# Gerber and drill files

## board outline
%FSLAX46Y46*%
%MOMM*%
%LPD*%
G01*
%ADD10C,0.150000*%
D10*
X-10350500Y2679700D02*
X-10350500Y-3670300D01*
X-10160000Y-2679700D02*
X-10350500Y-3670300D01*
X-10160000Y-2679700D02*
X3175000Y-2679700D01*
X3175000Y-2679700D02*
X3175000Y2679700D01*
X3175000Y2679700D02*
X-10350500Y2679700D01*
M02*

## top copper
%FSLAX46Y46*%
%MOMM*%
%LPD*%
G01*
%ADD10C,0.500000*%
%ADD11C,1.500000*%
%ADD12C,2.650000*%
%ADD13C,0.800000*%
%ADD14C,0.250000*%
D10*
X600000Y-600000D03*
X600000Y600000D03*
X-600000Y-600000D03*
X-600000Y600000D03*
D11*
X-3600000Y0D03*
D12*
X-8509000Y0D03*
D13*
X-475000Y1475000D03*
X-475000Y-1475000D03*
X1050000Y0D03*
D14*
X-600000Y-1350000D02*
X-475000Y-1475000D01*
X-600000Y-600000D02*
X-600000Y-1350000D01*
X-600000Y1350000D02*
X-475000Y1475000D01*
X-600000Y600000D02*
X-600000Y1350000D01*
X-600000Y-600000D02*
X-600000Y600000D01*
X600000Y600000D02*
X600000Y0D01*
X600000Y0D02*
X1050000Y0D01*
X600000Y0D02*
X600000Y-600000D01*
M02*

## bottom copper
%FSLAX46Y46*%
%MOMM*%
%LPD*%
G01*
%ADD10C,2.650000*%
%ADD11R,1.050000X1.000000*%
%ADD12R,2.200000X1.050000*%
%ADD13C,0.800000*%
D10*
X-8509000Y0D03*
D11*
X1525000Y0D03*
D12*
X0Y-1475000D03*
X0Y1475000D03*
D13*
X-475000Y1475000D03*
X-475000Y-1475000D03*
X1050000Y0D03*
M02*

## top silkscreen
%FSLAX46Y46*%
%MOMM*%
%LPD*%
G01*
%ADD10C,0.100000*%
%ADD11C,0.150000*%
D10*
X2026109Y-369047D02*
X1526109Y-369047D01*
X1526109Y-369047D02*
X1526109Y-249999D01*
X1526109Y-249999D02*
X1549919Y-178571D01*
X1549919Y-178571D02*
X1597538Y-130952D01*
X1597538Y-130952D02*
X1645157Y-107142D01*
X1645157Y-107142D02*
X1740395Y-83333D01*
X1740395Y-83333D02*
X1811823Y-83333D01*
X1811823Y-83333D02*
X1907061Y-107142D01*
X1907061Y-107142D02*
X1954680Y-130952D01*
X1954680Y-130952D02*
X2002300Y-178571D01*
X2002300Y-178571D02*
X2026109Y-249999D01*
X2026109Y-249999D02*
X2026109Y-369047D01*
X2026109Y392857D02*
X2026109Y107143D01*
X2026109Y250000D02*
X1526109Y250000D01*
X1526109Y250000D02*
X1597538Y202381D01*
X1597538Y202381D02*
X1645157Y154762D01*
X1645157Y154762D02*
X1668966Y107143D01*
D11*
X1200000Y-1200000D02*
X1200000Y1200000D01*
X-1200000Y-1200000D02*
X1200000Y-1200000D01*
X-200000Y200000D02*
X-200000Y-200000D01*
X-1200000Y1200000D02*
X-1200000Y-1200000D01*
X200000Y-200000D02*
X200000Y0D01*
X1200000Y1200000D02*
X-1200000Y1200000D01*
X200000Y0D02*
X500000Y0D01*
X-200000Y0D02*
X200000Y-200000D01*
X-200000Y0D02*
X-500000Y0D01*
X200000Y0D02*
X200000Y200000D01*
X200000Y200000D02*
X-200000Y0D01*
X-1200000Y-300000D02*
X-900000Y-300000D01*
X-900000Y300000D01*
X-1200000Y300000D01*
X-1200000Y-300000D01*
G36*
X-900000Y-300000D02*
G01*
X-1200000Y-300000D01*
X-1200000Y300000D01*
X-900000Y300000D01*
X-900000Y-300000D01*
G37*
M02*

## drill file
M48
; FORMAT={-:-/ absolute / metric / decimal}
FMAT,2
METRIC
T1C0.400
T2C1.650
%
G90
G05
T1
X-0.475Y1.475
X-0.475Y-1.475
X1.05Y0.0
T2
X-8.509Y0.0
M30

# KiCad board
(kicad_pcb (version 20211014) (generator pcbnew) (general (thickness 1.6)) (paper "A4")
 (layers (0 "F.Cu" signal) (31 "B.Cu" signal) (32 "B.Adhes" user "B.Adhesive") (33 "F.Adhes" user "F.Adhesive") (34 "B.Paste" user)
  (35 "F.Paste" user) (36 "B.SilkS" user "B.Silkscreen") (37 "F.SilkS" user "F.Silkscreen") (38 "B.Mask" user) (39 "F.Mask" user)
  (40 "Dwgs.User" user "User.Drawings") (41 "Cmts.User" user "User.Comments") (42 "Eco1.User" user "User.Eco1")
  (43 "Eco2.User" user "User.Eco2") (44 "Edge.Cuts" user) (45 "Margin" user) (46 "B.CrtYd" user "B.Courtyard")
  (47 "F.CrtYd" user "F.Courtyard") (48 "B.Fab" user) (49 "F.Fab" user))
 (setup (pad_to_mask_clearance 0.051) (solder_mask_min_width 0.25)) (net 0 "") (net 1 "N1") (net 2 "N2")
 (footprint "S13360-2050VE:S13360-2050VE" (layer "F.Cu") (at 0 0 -90)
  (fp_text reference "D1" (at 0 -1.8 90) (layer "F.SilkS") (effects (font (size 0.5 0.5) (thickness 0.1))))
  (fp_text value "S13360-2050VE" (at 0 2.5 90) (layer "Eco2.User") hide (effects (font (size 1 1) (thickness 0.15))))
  (fp_line (start 1.2 -1.2) (end -1.2 -1.2) (layer "F.SilkS") (width 0.15))
  (fp_line (start 1.2 1.2) (end 1.2 -1.2) (layer "F.SilkS") (width 0.15))
  (fp_line (start -0.2 0.2) (end 0.2 0.2) (layer "F.SilkS") (width 0.15))
  (fp_line (start -1.2 1.2) (end 1.2 1.2) (layer "F.SilkS") (width 0.15))
  (fp_line (start 0.2 -0.2) (end 0 -0.2) (layer "F.SilkS") (width 0.15))
  (fp_line (start -1.2 -1.2) (end -1.2 1.2) (layer "F.SilkS") (width 0.15))
  (fp_line (start 0 -0.2) (end 0 -0.5) (layer "F.SilkS") (width 0.15))
  (fp_line (start 0 0.2) (end 0.2 -0.2) (layer "F.SilkS") (width 0.15))
  (fp_line (start 0 0.2) (end 0 0.5) (layer "F.SilkS") (width 0.15))
  (fp_line (start 0 -0.2) (end -0.2 -0.2) (layer "F.SilkS") (width 0.15))
  (fp_line (start -0.2 -0.2) (end 0 0.2) (layer "F.SilkS") (width 0.15))
  (fp_poly (pts (xy 0.3 1.2) (xy 0.3 0.9) (xy -0.3 0.9) (xy -0.3 1.2)) (layer "F.SilkS") (width 0.15) (fill solid))
  (pad "1" smd circle locked (at 0.6 -0.6 270) (size 0.5 0.5) (layers "F.Cu" "F.Paste" "F.Mask"))
  (pad "1" smd circle locked (at -0.6 -0.6 270) (size 0.5 0.5) (layers "F.Cu" "F.Paste" "F.Mask"))
  (pad "2" smd circle locked (at 0.6 0.6 270) (size 0.5 0.5) (layers "F.Cu" "F.Paste" "F.Mask"))
  (pad "2" smd circle locked (at -0.6 0.6 270) (size 0.5 0.5) (layers "F.Cu" "F.Paste" "F.Mask")))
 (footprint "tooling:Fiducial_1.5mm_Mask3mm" (layer "F.Cu") (at -3.6 0)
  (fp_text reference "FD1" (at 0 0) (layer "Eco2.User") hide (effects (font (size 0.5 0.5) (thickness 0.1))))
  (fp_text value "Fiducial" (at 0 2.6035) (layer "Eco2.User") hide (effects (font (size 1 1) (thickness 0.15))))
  (pad "" smd circle locked (at 0 0) (size 1.5 1.5) (layers "F.Cu" "F.Mask") (solder_mask_margin 0.75) (clearance 0.75)))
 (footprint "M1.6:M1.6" (layer "B.Cu") (at -8.509 0 180)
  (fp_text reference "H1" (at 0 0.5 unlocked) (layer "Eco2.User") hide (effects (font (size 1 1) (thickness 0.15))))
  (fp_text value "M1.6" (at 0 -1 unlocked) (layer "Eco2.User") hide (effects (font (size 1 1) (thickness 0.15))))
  (pad "1" thru_hole circle (at 0 0 180) (size 2.65 2.65) (drill 1.65) (layers *.Cu *.Mask)))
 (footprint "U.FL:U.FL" (layer "B.Cu") (at 0 0 180)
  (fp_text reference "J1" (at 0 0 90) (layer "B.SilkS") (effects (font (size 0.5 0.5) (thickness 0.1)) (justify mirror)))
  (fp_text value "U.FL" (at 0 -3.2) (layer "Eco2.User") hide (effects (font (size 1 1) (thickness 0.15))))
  (pad "1" smd rect locked (at -1.525 0 180) (size 1.05 1) (layers "B.Cu" "B.Paste" "B.Mask") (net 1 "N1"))
  (pad "2" smd rect locked (at 0 -1.475 180) (size 2.2 1.05) (layers "B.Cu" "B.Paste" "B.Mask") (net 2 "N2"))
  (pad "2" smd rect locked (at 0 1.475 180) (size 2.2 1.05) (layers "B.Cu" "B.Paste" "B.Mask") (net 2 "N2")))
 (gr_line (start -10.3505 -2.6797) (end -10.3505 3.6703) (layer "Edge.Cuts") (width 0.15))
 (gr_line (start -10.16 2.6797) (end -10.3505 3.6703) (layer "Edge.Cuts") (width 0.15))
 (gr_line (start -10.16 2.6797) (end 3.175 2.6797) (layer "Edge.Cuts") (width 0.15))
 (gr_line (start 3.175 2.6797) (end 3.175 -2.6797) (layer "Edge.Cuts") (width 0.15))
 (gr_line (start 3.175 -2.6797) (end -10.3505 -2.6797) (layer "Edge.Cuts") (width 0.15))
 (segment (start -0.6 1.35) (end -0.475 1.475) (width 0.25) (layer "F.Cu") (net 2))
 (segment (start -0.6 0.6) (end -0.6 1.35) (width 0.25) (layer "F.Cu") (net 2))
 (segment (start -0.6 -1.35) (end -0.475 -1.475) (width 0.25) (layer "F.Cu") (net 2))
 (segment (start -0.6 -0.6) (end -0.6 -1.35) (width 0.25) (layer "F.Cu") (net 2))
 (segment (start -0.6 0.6) (end -0.6 -0.6) (width 0.25) (layer "F.Cu") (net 2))
 (via (at -0.475 -1.475) (size 0.8) (drill 0.4) (layers "F.Cu" "B.Cu") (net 2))
 (via (at -0.475 1.475) (size 0.8) (drill 0.4) (layers "F.Cu" "B.Cu") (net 2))
 (segment (start 0.6 -0.6) (end 0.6 0) (width 0.25) (layer "F.Cu") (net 1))
 (segment (start 0.6 0) (end 1.05 0) (width 0.25) (layer "F.Cu") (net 1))
 (segment (start 0.6 0) (end 0.6 0.6) (width 0.25) (layer "F.Cu") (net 1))
 (via (at 1.05 0) (size 0.8) (drill 0.4) (layers "F.Cu" "B.Cu") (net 1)))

